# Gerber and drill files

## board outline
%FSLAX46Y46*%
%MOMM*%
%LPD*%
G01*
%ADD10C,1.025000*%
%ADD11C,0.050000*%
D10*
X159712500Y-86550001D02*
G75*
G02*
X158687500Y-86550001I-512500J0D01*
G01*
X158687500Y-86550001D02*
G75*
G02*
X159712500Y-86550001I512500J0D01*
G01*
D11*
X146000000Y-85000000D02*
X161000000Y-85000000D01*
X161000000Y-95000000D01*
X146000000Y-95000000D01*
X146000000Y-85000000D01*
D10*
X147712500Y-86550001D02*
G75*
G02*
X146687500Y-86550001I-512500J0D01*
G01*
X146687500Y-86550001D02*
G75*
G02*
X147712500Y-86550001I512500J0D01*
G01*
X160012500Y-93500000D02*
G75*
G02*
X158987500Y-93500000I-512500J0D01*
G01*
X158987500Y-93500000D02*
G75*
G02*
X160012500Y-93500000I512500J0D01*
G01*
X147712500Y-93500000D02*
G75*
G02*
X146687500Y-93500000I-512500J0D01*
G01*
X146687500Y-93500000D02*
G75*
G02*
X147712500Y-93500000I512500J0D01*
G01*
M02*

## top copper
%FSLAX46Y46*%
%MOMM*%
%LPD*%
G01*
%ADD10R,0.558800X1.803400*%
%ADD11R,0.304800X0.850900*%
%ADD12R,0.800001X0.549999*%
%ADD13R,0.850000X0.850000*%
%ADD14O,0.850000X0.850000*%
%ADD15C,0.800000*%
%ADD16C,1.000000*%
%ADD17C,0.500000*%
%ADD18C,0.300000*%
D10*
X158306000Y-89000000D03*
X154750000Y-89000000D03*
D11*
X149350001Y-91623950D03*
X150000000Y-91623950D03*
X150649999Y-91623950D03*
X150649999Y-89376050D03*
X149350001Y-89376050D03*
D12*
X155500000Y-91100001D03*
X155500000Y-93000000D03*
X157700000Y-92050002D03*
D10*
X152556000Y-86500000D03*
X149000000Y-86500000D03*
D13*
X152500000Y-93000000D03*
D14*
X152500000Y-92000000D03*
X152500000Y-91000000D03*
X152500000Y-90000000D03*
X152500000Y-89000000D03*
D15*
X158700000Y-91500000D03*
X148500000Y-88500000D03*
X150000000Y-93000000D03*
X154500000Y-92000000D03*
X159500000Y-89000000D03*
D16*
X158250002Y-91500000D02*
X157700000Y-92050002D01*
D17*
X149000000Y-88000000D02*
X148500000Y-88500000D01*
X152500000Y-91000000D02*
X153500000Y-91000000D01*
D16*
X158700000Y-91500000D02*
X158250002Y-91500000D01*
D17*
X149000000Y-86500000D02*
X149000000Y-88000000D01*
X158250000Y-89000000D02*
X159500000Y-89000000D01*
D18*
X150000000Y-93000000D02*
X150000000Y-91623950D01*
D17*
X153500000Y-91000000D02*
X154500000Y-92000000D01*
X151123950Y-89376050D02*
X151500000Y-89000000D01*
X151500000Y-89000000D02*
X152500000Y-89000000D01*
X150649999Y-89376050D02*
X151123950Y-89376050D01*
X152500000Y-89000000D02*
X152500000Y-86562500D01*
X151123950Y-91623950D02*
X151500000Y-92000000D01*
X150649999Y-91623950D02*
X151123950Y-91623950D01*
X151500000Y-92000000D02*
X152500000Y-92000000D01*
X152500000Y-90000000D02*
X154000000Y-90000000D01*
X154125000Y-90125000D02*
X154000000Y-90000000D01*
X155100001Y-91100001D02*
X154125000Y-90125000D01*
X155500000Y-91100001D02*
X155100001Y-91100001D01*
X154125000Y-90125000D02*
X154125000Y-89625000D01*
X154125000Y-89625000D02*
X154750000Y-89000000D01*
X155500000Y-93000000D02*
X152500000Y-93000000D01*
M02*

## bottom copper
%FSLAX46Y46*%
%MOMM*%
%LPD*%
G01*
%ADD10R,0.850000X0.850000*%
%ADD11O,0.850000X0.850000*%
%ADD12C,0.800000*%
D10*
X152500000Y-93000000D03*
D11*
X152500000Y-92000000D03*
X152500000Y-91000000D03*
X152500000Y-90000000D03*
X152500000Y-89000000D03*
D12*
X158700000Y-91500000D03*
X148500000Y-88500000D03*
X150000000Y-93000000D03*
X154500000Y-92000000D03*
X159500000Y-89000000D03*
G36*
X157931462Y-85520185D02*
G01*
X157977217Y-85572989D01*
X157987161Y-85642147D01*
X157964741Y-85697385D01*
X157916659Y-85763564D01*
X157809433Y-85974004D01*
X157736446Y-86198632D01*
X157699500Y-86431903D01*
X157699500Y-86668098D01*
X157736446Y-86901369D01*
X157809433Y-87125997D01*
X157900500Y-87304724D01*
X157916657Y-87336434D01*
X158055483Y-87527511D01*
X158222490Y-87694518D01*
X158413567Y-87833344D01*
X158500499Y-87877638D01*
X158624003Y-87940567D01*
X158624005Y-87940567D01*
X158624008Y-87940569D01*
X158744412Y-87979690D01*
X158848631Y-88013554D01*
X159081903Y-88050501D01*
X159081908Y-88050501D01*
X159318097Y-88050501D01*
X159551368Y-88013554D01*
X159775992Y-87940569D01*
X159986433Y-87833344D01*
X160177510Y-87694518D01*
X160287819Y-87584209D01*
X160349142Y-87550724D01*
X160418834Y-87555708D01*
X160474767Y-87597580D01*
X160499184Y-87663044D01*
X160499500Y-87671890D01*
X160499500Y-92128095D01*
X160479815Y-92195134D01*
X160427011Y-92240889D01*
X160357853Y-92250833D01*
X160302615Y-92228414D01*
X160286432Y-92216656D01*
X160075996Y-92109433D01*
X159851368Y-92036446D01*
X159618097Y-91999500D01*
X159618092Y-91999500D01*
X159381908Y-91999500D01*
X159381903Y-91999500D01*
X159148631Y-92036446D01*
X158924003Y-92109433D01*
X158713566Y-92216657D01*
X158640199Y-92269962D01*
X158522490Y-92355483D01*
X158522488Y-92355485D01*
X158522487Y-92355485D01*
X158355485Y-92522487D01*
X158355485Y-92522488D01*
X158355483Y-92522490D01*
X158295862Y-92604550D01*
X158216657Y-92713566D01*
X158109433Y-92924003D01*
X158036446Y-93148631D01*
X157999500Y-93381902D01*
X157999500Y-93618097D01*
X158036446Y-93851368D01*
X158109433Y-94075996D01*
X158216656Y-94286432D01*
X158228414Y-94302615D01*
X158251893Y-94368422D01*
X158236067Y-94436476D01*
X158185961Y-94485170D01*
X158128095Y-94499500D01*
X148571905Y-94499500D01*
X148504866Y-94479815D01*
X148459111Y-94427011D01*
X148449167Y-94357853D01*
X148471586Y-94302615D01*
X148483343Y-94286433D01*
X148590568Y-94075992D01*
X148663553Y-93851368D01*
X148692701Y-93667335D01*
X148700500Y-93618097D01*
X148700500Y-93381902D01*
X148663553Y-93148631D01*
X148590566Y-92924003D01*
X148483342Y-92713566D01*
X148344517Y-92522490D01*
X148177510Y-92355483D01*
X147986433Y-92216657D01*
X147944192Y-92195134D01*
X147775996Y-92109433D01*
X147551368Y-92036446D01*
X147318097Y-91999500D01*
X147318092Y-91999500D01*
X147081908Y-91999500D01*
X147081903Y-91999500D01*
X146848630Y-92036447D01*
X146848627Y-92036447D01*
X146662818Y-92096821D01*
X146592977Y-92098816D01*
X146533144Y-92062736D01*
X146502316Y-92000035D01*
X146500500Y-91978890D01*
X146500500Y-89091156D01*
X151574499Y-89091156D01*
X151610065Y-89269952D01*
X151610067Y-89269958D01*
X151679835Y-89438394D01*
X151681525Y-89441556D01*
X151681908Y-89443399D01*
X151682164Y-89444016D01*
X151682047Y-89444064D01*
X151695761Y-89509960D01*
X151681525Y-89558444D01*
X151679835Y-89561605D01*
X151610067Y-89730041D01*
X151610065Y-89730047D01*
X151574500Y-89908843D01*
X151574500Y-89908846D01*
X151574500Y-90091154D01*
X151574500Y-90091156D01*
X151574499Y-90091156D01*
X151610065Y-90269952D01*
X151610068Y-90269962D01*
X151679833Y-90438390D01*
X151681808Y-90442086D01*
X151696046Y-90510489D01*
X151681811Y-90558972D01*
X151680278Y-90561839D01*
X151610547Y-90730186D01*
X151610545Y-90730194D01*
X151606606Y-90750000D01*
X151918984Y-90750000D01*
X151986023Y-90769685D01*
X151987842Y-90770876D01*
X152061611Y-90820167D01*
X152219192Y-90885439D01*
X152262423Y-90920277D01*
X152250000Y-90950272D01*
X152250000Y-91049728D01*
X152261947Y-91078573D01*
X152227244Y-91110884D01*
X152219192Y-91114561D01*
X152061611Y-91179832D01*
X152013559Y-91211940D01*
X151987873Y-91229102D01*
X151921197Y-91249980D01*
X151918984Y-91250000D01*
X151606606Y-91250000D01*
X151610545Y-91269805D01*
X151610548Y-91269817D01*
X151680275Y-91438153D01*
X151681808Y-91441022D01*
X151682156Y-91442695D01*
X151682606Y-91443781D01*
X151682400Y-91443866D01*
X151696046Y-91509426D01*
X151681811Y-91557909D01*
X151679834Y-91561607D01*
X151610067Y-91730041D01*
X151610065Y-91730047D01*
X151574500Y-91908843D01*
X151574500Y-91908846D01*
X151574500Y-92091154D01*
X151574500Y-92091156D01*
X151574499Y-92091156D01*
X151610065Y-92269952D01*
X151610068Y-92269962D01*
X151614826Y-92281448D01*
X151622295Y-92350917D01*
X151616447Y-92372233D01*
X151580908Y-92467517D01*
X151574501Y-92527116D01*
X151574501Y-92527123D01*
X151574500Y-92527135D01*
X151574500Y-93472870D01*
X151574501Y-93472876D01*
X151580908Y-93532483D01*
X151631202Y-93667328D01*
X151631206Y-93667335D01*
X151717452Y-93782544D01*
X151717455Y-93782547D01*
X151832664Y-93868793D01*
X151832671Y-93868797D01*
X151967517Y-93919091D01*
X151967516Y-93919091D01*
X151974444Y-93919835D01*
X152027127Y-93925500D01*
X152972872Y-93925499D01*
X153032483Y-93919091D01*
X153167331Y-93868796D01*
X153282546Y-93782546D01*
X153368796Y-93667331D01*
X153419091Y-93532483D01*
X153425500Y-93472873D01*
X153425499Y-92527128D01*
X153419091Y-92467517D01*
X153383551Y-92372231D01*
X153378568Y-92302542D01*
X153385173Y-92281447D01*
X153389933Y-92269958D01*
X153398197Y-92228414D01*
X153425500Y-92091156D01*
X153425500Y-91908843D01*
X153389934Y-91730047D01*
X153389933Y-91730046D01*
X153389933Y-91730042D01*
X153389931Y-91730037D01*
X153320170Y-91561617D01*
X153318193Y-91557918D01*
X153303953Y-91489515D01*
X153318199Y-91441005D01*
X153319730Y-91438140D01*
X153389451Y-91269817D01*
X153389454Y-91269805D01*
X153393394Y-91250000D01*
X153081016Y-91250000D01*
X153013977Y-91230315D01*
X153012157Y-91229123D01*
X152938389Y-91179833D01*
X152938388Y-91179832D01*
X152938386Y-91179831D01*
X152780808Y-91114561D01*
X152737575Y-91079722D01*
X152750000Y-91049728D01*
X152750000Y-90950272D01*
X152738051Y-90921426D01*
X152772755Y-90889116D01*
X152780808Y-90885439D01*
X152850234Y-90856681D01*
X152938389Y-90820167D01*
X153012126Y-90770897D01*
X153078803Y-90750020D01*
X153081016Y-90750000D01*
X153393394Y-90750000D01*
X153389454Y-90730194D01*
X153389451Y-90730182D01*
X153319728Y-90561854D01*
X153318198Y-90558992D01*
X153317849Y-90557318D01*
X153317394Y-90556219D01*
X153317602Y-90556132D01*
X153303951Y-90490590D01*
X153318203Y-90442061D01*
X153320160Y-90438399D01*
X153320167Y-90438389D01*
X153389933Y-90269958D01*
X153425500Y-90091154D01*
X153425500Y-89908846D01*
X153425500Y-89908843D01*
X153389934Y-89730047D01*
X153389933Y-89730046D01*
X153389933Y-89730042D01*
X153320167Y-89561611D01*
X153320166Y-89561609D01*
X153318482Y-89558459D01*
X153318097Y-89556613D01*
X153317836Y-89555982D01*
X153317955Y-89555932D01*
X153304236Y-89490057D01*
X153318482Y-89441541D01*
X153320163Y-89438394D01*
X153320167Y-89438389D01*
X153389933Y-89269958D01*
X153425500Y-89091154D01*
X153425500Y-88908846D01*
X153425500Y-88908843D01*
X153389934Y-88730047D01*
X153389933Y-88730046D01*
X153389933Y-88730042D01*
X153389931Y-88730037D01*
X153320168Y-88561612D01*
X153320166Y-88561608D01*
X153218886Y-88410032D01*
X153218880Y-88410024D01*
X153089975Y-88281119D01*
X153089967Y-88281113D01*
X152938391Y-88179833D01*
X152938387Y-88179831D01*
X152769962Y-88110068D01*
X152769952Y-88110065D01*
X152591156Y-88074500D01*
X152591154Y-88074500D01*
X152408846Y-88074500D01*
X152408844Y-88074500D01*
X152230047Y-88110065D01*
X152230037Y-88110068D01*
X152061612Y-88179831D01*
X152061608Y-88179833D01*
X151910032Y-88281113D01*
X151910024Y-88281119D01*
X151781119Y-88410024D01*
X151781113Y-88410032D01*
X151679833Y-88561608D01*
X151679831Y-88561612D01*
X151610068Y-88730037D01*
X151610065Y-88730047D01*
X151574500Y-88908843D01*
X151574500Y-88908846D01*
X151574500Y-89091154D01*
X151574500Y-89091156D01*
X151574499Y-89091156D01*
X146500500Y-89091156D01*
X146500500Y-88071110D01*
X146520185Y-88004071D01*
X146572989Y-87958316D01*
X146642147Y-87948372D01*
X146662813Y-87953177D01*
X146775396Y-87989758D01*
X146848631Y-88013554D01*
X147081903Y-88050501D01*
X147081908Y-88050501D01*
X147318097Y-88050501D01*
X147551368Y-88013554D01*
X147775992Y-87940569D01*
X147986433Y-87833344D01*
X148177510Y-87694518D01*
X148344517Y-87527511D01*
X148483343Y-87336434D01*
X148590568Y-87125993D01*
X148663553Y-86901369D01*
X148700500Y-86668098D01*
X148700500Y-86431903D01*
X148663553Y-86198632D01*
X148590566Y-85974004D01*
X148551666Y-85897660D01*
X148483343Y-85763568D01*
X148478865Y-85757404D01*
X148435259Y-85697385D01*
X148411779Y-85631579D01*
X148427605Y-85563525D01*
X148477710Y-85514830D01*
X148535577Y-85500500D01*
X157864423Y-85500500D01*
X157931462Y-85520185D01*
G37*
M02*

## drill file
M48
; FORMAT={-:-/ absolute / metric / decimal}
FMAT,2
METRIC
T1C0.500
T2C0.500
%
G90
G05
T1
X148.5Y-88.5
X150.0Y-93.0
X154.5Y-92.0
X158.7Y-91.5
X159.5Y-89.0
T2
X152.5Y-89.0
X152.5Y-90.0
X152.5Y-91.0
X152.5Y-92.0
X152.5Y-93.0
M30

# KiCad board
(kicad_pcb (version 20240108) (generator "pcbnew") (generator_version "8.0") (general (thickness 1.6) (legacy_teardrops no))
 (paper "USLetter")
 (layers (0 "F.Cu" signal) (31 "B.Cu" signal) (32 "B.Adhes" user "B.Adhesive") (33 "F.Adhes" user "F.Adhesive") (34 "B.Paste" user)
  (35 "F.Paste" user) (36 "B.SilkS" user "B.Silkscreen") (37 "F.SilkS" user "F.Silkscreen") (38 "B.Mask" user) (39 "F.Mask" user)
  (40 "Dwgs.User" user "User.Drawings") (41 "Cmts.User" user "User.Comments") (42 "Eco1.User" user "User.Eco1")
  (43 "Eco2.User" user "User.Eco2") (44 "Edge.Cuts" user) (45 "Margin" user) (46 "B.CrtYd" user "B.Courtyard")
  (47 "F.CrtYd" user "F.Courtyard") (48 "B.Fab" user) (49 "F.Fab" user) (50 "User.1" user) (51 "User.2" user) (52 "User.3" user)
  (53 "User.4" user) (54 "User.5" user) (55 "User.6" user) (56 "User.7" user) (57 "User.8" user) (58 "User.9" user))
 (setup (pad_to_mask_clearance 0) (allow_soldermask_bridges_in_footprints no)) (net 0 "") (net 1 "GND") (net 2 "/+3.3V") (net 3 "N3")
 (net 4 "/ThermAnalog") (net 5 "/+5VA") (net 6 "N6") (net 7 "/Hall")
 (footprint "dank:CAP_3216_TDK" (layer "F.Cu") (at 156.528 89 180)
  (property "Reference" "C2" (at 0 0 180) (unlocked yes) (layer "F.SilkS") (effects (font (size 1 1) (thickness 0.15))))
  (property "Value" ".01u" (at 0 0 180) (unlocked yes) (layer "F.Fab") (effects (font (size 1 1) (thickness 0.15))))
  (pad "1" smd rect (at -1.778 0 180) (size 0.5588 1.8034) (layers "F.Cu" "F.Paste" "F.Mask") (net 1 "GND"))
  (pad "2" smd rect (at 1.778 0 180) (size 0.5588 1.8034) (layers "F.Cu" "F.Paste" "F.Mask") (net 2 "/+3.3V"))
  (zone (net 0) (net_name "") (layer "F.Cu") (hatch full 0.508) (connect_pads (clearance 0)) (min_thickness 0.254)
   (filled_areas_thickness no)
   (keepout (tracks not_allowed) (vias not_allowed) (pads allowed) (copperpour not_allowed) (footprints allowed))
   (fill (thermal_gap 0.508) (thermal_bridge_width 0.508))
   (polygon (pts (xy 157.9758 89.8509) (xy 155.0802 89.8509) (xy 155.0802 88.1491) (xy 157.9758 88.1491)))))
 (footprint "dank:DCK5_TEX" (layer "F.Cu") (at 150 90.5 90)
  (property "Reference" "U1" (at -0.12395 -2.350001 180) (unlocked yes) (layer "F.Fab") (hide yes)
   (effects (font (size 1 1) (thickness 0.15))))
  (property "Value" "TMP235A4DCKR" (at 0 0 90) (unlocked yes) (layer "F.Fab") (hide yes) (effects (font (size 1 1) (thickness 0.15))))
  (pad "1" smd rect (at -1.12395 -0.649999 90) (size 0.8509 0.3048) (layers "F.Cu" "F.Paste" "F.Mask") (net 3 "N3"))
  (pad "2" smd rect (at -1.12395 0 90) (size 0.8509 0.3048) (layers "F.Cu" "F.Paste" "F.Mask") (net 1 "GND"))
  (pad "3" smd rect (at -1.12395 0.649999 90) (size 0.8509 0.3048) (layers "F.Cu" "F.Paste" "F.Mask") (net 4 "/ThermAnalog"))
  (pad "4" smd rect (at 1.12395 0.649999 90) (size 0.8509 0.3048) (layers "F.Cu" "F.Paste" "F.Mask") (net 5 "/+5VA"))
  (pad "5" smd rect (at 1.12395 -0.649999 90) (size 0.8509 0.3048) (layers "F.Cu" "F.Paste" "F.Mask") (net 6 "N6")))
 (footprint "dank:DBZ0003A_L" (layer "F.Cu") (at 156.6 92.050002)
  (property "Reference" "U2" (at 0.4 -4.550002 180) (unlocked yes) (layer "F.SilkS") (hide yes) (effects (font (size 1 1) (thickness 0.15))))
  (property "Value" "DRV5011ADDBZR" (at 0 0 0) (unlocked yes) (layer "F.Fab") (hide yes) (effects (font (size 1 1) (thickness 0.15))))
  (pad "1" smd rect (at -1.1 -0.950001 90) (size 0.549999 0.800001) (layers "F.Cu" "F.Paste" "F.Mask") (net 2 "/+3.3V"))
  (pad "2" smd rect (at -1.1 0.949998 90) (size 0.549999 0.800001) (layers "F.Cu" "F.Paste" "F.Mask") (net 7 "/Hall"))
  (pad "3" smd rect (at 1.1 0 90) (size 0.549999 0.800001) (layers "F.Cu" "F.Paste" "F.Mask") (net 1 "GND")))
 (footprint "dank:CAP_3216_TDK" (layer "F.Cu") (at 150.778 86.5 180)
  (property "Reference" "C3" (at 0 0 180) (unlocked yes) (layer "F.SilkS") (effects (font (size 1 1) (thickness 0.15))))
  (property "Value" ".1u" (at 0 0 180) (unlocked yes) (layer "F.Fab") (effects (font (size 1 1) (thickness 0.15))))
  (pad "1" smd rect (at -1.778 0 180) (size 0.5588 1.8034) (layers "F.Cu" "F.Paste" "F.Mask") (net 5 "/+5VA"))
  (pad "2" smd rect (at 1.778 0 180) (size 0.5588 1.8034) (layers "F.Cu" "F.Paste" "F.Mask") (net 1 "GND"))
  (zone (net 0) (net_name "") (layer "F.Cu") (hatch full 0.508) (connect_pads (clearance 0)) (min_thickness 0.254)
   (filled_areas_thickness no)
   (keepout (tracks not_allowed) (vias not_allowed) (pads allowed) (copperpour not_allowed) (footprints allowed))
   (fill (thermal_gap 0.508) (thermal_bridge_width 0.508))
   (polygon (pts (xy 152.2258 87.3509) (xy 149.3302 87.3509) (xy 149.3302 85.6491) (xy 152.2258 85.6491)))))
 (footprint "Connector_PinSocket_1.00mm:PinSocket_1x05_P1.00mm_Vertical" (layer "F.Cu") (at 152.5 93 180)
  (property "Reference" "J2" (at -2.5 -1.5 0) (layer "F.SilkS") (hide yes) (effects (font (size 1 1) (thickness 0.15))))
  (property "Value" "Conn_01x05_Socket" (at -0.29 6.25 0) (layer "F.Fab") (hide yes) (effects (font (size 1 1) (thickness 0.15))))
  (pad "1" thru_hole rect (at 0 0 180) (size 0.85 0.85) (drill 0.5) (layers "*.Cu" "*.Mask") (remove_unused_layers no) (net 7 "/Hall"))
  (pad "2" thru_hole oval (at 0 1 180) (size 0.85 0.85) (drill 0.5) (layers "*.Cu" "*.Mask") (remove_unused_layers no)
   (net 4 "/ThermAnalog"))
  (pad "3" thru_hole oval (at 0 2 180) (size 0.85 0.85) (drill 0.5) (layers "*.Cu" "*.Mask") (remove_unused_layers no) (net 1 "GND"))
  (pad "4" thru_hole oval (at 0 3 180) (size 0.85 0.85) (drill 0.5) (layers "*.Cu" "*.Mask") (remove_unused_layers no) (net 2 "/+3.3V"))
  (pad "5" thru_hole oval (at 0 4 180) (size 0.85 0.85) (drill 0.5) (layers "*.Cu" "*.Mask") (remove_unused_layers no) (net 5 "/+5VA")))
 (gr_circle (center 159.2 86.550001) (end 160.2 86.550001) (stroke (width 0.05) (type default)) (fill solid) (layer "Edge.Cuts"))
 (gr_rect (start 146 85) (end 161 95) (stroke (width 0.05) (type default)) (fill none) (layer "Edge.Cuts"))
 (gr_circle (center 147.2 86.550001) (end 148.2 86.550001) (stroke (width 0.05) (type default)) (fill solid) (layer "Edge.Cuts"))
 (gr_circle (center 159.5 93.5) (end 160.5 93.5) (stroke (width 0.05) (type default)) (fill solid) (layer "Edge.Cuts"))
 (gr_circle (center 147.2 93.5) (end 148.2 93.5) (stroke (width 0.05) (type default)) (fill solid) (layer "Edge.Cuts"))
 (segment (start 158.250002 91.5) (end 157.7 92.050002) (width 1) (layer "F.Cu") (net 1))
 (segment (start 149 88) (end 148.5 88.5) (width 0.5) (layer "F.Cu") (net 1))
 (segment (start 152.5 91) (end 153.5 91) (width 0.5) (layer "F.Cu") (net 1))
 (segment (start 158.7 91.5) (end 158.250002 91.5) (width 1) (layer "F.Cu") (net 1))
 (segment (start 149 86.5) (end 149 88) (width 0.5) (layer "F.Cu") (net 1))
 (segment (start 158.25 89) (end 159.5 89) (width 0.5) (layer "F.Cu") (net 1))
 (segment (start 150 93) (end 150 91.62395) (width 0.3) (layer "F.Cu") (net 1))
 (segment (start 153.5 91) (end 154.5 92) (width 0.5) (layer "F.Cu") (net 1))
 (via (at 158.7 91.5) (size 0.8) (drill 0.5) (layers "F.Cu" "B.Cu") (free yes) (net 1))
 (via (at 148.5 88.5) (size 0.8) (drill 0.5) (layers "F.Cu" "B.Cu") (free yes) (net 1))
 (via (at 150 93) (size 0.8) (drill 0.5) (layers "F.Cu" "B.Cu") (free yes) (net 1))
 (via (at 154.5 92) (size 0.8) (drill 0.5) (layers "F.Cu" "B.Cu") (free yes) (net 1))
 (via (at 159.5 89) (size 0.8) (drill 0.5) (layers "F.Cu" "B.Cu") (free yes) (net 1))
 (segment (start 151.12395 89.37605) (end 151.5 89) (width 0.5) (layer "F.Cu") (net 5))
 (segment (start 151.5 89) (end 152.5 89) (width 0.5) (layer "F.Cu") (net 5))
 (segment (start 150.649999 89.37605) (end 151.12395 89.37605) (width 0.5) (layer "F.Cu") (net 5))
 (segment (start 152.5 89) (end 152.5 86.5625) (width 0.5) (layer "F.Cu") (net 5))
 (segment (start 151.12395 91.62395) (end 151.5 92) (width 0.5) (layer "F.Cu") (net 4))
 (segment (start 150.649999 91.62395) (end 151.12395 91.62395) (width 0.5) (layer "F.Cu") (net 4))
 (segment (start 151.5 92) (end 152.5 92) (width 0.5) (layer "F.Cu") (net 4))
 (segment (start 152.5 90) (end 154 90) (width 0.5) (layer "F.Cu") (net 2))
 (segment (start 154.125 90.125) (end 154 90) (width 0.5) (layer "F.Cu") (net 2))
 (segment (start 155.100001 91.100001) (end 154.125 90.125) (width 0.5) (layer "F.Cu") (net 2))
 (segment (start 155.5 91.100001) (end 155.100001 91.100001) (width 0.5) (layer "F.Cu") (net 2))
 (segment (start 154.125 90.125) (end 154.125 89.625) (width 0.5) (layer "F.Cu") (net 2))
 (segment (start 154.125 89.625) (end 154.75 89) (width 0.5) (layer "F.Cu") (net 2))
 (segment (start 155.5 93) (end 152.5 93) (width 0.5) (layer "F.Cu") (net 7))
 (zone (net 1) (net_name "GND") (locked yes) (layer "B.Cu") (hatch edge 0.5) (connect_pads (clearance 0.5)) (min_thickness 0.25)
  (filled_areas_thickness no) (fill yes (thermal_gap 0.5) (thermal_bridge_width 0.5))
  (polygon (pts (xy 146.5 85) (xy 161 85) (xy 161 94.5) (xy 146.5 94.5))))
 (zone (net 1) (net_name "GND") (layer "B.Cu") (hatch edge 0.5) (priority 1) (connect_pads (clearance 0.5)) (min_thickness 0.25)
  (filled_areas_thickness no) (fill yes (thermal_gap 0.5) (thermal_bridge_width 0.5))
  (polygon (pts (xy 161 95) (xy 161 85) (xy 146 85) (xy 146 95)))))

